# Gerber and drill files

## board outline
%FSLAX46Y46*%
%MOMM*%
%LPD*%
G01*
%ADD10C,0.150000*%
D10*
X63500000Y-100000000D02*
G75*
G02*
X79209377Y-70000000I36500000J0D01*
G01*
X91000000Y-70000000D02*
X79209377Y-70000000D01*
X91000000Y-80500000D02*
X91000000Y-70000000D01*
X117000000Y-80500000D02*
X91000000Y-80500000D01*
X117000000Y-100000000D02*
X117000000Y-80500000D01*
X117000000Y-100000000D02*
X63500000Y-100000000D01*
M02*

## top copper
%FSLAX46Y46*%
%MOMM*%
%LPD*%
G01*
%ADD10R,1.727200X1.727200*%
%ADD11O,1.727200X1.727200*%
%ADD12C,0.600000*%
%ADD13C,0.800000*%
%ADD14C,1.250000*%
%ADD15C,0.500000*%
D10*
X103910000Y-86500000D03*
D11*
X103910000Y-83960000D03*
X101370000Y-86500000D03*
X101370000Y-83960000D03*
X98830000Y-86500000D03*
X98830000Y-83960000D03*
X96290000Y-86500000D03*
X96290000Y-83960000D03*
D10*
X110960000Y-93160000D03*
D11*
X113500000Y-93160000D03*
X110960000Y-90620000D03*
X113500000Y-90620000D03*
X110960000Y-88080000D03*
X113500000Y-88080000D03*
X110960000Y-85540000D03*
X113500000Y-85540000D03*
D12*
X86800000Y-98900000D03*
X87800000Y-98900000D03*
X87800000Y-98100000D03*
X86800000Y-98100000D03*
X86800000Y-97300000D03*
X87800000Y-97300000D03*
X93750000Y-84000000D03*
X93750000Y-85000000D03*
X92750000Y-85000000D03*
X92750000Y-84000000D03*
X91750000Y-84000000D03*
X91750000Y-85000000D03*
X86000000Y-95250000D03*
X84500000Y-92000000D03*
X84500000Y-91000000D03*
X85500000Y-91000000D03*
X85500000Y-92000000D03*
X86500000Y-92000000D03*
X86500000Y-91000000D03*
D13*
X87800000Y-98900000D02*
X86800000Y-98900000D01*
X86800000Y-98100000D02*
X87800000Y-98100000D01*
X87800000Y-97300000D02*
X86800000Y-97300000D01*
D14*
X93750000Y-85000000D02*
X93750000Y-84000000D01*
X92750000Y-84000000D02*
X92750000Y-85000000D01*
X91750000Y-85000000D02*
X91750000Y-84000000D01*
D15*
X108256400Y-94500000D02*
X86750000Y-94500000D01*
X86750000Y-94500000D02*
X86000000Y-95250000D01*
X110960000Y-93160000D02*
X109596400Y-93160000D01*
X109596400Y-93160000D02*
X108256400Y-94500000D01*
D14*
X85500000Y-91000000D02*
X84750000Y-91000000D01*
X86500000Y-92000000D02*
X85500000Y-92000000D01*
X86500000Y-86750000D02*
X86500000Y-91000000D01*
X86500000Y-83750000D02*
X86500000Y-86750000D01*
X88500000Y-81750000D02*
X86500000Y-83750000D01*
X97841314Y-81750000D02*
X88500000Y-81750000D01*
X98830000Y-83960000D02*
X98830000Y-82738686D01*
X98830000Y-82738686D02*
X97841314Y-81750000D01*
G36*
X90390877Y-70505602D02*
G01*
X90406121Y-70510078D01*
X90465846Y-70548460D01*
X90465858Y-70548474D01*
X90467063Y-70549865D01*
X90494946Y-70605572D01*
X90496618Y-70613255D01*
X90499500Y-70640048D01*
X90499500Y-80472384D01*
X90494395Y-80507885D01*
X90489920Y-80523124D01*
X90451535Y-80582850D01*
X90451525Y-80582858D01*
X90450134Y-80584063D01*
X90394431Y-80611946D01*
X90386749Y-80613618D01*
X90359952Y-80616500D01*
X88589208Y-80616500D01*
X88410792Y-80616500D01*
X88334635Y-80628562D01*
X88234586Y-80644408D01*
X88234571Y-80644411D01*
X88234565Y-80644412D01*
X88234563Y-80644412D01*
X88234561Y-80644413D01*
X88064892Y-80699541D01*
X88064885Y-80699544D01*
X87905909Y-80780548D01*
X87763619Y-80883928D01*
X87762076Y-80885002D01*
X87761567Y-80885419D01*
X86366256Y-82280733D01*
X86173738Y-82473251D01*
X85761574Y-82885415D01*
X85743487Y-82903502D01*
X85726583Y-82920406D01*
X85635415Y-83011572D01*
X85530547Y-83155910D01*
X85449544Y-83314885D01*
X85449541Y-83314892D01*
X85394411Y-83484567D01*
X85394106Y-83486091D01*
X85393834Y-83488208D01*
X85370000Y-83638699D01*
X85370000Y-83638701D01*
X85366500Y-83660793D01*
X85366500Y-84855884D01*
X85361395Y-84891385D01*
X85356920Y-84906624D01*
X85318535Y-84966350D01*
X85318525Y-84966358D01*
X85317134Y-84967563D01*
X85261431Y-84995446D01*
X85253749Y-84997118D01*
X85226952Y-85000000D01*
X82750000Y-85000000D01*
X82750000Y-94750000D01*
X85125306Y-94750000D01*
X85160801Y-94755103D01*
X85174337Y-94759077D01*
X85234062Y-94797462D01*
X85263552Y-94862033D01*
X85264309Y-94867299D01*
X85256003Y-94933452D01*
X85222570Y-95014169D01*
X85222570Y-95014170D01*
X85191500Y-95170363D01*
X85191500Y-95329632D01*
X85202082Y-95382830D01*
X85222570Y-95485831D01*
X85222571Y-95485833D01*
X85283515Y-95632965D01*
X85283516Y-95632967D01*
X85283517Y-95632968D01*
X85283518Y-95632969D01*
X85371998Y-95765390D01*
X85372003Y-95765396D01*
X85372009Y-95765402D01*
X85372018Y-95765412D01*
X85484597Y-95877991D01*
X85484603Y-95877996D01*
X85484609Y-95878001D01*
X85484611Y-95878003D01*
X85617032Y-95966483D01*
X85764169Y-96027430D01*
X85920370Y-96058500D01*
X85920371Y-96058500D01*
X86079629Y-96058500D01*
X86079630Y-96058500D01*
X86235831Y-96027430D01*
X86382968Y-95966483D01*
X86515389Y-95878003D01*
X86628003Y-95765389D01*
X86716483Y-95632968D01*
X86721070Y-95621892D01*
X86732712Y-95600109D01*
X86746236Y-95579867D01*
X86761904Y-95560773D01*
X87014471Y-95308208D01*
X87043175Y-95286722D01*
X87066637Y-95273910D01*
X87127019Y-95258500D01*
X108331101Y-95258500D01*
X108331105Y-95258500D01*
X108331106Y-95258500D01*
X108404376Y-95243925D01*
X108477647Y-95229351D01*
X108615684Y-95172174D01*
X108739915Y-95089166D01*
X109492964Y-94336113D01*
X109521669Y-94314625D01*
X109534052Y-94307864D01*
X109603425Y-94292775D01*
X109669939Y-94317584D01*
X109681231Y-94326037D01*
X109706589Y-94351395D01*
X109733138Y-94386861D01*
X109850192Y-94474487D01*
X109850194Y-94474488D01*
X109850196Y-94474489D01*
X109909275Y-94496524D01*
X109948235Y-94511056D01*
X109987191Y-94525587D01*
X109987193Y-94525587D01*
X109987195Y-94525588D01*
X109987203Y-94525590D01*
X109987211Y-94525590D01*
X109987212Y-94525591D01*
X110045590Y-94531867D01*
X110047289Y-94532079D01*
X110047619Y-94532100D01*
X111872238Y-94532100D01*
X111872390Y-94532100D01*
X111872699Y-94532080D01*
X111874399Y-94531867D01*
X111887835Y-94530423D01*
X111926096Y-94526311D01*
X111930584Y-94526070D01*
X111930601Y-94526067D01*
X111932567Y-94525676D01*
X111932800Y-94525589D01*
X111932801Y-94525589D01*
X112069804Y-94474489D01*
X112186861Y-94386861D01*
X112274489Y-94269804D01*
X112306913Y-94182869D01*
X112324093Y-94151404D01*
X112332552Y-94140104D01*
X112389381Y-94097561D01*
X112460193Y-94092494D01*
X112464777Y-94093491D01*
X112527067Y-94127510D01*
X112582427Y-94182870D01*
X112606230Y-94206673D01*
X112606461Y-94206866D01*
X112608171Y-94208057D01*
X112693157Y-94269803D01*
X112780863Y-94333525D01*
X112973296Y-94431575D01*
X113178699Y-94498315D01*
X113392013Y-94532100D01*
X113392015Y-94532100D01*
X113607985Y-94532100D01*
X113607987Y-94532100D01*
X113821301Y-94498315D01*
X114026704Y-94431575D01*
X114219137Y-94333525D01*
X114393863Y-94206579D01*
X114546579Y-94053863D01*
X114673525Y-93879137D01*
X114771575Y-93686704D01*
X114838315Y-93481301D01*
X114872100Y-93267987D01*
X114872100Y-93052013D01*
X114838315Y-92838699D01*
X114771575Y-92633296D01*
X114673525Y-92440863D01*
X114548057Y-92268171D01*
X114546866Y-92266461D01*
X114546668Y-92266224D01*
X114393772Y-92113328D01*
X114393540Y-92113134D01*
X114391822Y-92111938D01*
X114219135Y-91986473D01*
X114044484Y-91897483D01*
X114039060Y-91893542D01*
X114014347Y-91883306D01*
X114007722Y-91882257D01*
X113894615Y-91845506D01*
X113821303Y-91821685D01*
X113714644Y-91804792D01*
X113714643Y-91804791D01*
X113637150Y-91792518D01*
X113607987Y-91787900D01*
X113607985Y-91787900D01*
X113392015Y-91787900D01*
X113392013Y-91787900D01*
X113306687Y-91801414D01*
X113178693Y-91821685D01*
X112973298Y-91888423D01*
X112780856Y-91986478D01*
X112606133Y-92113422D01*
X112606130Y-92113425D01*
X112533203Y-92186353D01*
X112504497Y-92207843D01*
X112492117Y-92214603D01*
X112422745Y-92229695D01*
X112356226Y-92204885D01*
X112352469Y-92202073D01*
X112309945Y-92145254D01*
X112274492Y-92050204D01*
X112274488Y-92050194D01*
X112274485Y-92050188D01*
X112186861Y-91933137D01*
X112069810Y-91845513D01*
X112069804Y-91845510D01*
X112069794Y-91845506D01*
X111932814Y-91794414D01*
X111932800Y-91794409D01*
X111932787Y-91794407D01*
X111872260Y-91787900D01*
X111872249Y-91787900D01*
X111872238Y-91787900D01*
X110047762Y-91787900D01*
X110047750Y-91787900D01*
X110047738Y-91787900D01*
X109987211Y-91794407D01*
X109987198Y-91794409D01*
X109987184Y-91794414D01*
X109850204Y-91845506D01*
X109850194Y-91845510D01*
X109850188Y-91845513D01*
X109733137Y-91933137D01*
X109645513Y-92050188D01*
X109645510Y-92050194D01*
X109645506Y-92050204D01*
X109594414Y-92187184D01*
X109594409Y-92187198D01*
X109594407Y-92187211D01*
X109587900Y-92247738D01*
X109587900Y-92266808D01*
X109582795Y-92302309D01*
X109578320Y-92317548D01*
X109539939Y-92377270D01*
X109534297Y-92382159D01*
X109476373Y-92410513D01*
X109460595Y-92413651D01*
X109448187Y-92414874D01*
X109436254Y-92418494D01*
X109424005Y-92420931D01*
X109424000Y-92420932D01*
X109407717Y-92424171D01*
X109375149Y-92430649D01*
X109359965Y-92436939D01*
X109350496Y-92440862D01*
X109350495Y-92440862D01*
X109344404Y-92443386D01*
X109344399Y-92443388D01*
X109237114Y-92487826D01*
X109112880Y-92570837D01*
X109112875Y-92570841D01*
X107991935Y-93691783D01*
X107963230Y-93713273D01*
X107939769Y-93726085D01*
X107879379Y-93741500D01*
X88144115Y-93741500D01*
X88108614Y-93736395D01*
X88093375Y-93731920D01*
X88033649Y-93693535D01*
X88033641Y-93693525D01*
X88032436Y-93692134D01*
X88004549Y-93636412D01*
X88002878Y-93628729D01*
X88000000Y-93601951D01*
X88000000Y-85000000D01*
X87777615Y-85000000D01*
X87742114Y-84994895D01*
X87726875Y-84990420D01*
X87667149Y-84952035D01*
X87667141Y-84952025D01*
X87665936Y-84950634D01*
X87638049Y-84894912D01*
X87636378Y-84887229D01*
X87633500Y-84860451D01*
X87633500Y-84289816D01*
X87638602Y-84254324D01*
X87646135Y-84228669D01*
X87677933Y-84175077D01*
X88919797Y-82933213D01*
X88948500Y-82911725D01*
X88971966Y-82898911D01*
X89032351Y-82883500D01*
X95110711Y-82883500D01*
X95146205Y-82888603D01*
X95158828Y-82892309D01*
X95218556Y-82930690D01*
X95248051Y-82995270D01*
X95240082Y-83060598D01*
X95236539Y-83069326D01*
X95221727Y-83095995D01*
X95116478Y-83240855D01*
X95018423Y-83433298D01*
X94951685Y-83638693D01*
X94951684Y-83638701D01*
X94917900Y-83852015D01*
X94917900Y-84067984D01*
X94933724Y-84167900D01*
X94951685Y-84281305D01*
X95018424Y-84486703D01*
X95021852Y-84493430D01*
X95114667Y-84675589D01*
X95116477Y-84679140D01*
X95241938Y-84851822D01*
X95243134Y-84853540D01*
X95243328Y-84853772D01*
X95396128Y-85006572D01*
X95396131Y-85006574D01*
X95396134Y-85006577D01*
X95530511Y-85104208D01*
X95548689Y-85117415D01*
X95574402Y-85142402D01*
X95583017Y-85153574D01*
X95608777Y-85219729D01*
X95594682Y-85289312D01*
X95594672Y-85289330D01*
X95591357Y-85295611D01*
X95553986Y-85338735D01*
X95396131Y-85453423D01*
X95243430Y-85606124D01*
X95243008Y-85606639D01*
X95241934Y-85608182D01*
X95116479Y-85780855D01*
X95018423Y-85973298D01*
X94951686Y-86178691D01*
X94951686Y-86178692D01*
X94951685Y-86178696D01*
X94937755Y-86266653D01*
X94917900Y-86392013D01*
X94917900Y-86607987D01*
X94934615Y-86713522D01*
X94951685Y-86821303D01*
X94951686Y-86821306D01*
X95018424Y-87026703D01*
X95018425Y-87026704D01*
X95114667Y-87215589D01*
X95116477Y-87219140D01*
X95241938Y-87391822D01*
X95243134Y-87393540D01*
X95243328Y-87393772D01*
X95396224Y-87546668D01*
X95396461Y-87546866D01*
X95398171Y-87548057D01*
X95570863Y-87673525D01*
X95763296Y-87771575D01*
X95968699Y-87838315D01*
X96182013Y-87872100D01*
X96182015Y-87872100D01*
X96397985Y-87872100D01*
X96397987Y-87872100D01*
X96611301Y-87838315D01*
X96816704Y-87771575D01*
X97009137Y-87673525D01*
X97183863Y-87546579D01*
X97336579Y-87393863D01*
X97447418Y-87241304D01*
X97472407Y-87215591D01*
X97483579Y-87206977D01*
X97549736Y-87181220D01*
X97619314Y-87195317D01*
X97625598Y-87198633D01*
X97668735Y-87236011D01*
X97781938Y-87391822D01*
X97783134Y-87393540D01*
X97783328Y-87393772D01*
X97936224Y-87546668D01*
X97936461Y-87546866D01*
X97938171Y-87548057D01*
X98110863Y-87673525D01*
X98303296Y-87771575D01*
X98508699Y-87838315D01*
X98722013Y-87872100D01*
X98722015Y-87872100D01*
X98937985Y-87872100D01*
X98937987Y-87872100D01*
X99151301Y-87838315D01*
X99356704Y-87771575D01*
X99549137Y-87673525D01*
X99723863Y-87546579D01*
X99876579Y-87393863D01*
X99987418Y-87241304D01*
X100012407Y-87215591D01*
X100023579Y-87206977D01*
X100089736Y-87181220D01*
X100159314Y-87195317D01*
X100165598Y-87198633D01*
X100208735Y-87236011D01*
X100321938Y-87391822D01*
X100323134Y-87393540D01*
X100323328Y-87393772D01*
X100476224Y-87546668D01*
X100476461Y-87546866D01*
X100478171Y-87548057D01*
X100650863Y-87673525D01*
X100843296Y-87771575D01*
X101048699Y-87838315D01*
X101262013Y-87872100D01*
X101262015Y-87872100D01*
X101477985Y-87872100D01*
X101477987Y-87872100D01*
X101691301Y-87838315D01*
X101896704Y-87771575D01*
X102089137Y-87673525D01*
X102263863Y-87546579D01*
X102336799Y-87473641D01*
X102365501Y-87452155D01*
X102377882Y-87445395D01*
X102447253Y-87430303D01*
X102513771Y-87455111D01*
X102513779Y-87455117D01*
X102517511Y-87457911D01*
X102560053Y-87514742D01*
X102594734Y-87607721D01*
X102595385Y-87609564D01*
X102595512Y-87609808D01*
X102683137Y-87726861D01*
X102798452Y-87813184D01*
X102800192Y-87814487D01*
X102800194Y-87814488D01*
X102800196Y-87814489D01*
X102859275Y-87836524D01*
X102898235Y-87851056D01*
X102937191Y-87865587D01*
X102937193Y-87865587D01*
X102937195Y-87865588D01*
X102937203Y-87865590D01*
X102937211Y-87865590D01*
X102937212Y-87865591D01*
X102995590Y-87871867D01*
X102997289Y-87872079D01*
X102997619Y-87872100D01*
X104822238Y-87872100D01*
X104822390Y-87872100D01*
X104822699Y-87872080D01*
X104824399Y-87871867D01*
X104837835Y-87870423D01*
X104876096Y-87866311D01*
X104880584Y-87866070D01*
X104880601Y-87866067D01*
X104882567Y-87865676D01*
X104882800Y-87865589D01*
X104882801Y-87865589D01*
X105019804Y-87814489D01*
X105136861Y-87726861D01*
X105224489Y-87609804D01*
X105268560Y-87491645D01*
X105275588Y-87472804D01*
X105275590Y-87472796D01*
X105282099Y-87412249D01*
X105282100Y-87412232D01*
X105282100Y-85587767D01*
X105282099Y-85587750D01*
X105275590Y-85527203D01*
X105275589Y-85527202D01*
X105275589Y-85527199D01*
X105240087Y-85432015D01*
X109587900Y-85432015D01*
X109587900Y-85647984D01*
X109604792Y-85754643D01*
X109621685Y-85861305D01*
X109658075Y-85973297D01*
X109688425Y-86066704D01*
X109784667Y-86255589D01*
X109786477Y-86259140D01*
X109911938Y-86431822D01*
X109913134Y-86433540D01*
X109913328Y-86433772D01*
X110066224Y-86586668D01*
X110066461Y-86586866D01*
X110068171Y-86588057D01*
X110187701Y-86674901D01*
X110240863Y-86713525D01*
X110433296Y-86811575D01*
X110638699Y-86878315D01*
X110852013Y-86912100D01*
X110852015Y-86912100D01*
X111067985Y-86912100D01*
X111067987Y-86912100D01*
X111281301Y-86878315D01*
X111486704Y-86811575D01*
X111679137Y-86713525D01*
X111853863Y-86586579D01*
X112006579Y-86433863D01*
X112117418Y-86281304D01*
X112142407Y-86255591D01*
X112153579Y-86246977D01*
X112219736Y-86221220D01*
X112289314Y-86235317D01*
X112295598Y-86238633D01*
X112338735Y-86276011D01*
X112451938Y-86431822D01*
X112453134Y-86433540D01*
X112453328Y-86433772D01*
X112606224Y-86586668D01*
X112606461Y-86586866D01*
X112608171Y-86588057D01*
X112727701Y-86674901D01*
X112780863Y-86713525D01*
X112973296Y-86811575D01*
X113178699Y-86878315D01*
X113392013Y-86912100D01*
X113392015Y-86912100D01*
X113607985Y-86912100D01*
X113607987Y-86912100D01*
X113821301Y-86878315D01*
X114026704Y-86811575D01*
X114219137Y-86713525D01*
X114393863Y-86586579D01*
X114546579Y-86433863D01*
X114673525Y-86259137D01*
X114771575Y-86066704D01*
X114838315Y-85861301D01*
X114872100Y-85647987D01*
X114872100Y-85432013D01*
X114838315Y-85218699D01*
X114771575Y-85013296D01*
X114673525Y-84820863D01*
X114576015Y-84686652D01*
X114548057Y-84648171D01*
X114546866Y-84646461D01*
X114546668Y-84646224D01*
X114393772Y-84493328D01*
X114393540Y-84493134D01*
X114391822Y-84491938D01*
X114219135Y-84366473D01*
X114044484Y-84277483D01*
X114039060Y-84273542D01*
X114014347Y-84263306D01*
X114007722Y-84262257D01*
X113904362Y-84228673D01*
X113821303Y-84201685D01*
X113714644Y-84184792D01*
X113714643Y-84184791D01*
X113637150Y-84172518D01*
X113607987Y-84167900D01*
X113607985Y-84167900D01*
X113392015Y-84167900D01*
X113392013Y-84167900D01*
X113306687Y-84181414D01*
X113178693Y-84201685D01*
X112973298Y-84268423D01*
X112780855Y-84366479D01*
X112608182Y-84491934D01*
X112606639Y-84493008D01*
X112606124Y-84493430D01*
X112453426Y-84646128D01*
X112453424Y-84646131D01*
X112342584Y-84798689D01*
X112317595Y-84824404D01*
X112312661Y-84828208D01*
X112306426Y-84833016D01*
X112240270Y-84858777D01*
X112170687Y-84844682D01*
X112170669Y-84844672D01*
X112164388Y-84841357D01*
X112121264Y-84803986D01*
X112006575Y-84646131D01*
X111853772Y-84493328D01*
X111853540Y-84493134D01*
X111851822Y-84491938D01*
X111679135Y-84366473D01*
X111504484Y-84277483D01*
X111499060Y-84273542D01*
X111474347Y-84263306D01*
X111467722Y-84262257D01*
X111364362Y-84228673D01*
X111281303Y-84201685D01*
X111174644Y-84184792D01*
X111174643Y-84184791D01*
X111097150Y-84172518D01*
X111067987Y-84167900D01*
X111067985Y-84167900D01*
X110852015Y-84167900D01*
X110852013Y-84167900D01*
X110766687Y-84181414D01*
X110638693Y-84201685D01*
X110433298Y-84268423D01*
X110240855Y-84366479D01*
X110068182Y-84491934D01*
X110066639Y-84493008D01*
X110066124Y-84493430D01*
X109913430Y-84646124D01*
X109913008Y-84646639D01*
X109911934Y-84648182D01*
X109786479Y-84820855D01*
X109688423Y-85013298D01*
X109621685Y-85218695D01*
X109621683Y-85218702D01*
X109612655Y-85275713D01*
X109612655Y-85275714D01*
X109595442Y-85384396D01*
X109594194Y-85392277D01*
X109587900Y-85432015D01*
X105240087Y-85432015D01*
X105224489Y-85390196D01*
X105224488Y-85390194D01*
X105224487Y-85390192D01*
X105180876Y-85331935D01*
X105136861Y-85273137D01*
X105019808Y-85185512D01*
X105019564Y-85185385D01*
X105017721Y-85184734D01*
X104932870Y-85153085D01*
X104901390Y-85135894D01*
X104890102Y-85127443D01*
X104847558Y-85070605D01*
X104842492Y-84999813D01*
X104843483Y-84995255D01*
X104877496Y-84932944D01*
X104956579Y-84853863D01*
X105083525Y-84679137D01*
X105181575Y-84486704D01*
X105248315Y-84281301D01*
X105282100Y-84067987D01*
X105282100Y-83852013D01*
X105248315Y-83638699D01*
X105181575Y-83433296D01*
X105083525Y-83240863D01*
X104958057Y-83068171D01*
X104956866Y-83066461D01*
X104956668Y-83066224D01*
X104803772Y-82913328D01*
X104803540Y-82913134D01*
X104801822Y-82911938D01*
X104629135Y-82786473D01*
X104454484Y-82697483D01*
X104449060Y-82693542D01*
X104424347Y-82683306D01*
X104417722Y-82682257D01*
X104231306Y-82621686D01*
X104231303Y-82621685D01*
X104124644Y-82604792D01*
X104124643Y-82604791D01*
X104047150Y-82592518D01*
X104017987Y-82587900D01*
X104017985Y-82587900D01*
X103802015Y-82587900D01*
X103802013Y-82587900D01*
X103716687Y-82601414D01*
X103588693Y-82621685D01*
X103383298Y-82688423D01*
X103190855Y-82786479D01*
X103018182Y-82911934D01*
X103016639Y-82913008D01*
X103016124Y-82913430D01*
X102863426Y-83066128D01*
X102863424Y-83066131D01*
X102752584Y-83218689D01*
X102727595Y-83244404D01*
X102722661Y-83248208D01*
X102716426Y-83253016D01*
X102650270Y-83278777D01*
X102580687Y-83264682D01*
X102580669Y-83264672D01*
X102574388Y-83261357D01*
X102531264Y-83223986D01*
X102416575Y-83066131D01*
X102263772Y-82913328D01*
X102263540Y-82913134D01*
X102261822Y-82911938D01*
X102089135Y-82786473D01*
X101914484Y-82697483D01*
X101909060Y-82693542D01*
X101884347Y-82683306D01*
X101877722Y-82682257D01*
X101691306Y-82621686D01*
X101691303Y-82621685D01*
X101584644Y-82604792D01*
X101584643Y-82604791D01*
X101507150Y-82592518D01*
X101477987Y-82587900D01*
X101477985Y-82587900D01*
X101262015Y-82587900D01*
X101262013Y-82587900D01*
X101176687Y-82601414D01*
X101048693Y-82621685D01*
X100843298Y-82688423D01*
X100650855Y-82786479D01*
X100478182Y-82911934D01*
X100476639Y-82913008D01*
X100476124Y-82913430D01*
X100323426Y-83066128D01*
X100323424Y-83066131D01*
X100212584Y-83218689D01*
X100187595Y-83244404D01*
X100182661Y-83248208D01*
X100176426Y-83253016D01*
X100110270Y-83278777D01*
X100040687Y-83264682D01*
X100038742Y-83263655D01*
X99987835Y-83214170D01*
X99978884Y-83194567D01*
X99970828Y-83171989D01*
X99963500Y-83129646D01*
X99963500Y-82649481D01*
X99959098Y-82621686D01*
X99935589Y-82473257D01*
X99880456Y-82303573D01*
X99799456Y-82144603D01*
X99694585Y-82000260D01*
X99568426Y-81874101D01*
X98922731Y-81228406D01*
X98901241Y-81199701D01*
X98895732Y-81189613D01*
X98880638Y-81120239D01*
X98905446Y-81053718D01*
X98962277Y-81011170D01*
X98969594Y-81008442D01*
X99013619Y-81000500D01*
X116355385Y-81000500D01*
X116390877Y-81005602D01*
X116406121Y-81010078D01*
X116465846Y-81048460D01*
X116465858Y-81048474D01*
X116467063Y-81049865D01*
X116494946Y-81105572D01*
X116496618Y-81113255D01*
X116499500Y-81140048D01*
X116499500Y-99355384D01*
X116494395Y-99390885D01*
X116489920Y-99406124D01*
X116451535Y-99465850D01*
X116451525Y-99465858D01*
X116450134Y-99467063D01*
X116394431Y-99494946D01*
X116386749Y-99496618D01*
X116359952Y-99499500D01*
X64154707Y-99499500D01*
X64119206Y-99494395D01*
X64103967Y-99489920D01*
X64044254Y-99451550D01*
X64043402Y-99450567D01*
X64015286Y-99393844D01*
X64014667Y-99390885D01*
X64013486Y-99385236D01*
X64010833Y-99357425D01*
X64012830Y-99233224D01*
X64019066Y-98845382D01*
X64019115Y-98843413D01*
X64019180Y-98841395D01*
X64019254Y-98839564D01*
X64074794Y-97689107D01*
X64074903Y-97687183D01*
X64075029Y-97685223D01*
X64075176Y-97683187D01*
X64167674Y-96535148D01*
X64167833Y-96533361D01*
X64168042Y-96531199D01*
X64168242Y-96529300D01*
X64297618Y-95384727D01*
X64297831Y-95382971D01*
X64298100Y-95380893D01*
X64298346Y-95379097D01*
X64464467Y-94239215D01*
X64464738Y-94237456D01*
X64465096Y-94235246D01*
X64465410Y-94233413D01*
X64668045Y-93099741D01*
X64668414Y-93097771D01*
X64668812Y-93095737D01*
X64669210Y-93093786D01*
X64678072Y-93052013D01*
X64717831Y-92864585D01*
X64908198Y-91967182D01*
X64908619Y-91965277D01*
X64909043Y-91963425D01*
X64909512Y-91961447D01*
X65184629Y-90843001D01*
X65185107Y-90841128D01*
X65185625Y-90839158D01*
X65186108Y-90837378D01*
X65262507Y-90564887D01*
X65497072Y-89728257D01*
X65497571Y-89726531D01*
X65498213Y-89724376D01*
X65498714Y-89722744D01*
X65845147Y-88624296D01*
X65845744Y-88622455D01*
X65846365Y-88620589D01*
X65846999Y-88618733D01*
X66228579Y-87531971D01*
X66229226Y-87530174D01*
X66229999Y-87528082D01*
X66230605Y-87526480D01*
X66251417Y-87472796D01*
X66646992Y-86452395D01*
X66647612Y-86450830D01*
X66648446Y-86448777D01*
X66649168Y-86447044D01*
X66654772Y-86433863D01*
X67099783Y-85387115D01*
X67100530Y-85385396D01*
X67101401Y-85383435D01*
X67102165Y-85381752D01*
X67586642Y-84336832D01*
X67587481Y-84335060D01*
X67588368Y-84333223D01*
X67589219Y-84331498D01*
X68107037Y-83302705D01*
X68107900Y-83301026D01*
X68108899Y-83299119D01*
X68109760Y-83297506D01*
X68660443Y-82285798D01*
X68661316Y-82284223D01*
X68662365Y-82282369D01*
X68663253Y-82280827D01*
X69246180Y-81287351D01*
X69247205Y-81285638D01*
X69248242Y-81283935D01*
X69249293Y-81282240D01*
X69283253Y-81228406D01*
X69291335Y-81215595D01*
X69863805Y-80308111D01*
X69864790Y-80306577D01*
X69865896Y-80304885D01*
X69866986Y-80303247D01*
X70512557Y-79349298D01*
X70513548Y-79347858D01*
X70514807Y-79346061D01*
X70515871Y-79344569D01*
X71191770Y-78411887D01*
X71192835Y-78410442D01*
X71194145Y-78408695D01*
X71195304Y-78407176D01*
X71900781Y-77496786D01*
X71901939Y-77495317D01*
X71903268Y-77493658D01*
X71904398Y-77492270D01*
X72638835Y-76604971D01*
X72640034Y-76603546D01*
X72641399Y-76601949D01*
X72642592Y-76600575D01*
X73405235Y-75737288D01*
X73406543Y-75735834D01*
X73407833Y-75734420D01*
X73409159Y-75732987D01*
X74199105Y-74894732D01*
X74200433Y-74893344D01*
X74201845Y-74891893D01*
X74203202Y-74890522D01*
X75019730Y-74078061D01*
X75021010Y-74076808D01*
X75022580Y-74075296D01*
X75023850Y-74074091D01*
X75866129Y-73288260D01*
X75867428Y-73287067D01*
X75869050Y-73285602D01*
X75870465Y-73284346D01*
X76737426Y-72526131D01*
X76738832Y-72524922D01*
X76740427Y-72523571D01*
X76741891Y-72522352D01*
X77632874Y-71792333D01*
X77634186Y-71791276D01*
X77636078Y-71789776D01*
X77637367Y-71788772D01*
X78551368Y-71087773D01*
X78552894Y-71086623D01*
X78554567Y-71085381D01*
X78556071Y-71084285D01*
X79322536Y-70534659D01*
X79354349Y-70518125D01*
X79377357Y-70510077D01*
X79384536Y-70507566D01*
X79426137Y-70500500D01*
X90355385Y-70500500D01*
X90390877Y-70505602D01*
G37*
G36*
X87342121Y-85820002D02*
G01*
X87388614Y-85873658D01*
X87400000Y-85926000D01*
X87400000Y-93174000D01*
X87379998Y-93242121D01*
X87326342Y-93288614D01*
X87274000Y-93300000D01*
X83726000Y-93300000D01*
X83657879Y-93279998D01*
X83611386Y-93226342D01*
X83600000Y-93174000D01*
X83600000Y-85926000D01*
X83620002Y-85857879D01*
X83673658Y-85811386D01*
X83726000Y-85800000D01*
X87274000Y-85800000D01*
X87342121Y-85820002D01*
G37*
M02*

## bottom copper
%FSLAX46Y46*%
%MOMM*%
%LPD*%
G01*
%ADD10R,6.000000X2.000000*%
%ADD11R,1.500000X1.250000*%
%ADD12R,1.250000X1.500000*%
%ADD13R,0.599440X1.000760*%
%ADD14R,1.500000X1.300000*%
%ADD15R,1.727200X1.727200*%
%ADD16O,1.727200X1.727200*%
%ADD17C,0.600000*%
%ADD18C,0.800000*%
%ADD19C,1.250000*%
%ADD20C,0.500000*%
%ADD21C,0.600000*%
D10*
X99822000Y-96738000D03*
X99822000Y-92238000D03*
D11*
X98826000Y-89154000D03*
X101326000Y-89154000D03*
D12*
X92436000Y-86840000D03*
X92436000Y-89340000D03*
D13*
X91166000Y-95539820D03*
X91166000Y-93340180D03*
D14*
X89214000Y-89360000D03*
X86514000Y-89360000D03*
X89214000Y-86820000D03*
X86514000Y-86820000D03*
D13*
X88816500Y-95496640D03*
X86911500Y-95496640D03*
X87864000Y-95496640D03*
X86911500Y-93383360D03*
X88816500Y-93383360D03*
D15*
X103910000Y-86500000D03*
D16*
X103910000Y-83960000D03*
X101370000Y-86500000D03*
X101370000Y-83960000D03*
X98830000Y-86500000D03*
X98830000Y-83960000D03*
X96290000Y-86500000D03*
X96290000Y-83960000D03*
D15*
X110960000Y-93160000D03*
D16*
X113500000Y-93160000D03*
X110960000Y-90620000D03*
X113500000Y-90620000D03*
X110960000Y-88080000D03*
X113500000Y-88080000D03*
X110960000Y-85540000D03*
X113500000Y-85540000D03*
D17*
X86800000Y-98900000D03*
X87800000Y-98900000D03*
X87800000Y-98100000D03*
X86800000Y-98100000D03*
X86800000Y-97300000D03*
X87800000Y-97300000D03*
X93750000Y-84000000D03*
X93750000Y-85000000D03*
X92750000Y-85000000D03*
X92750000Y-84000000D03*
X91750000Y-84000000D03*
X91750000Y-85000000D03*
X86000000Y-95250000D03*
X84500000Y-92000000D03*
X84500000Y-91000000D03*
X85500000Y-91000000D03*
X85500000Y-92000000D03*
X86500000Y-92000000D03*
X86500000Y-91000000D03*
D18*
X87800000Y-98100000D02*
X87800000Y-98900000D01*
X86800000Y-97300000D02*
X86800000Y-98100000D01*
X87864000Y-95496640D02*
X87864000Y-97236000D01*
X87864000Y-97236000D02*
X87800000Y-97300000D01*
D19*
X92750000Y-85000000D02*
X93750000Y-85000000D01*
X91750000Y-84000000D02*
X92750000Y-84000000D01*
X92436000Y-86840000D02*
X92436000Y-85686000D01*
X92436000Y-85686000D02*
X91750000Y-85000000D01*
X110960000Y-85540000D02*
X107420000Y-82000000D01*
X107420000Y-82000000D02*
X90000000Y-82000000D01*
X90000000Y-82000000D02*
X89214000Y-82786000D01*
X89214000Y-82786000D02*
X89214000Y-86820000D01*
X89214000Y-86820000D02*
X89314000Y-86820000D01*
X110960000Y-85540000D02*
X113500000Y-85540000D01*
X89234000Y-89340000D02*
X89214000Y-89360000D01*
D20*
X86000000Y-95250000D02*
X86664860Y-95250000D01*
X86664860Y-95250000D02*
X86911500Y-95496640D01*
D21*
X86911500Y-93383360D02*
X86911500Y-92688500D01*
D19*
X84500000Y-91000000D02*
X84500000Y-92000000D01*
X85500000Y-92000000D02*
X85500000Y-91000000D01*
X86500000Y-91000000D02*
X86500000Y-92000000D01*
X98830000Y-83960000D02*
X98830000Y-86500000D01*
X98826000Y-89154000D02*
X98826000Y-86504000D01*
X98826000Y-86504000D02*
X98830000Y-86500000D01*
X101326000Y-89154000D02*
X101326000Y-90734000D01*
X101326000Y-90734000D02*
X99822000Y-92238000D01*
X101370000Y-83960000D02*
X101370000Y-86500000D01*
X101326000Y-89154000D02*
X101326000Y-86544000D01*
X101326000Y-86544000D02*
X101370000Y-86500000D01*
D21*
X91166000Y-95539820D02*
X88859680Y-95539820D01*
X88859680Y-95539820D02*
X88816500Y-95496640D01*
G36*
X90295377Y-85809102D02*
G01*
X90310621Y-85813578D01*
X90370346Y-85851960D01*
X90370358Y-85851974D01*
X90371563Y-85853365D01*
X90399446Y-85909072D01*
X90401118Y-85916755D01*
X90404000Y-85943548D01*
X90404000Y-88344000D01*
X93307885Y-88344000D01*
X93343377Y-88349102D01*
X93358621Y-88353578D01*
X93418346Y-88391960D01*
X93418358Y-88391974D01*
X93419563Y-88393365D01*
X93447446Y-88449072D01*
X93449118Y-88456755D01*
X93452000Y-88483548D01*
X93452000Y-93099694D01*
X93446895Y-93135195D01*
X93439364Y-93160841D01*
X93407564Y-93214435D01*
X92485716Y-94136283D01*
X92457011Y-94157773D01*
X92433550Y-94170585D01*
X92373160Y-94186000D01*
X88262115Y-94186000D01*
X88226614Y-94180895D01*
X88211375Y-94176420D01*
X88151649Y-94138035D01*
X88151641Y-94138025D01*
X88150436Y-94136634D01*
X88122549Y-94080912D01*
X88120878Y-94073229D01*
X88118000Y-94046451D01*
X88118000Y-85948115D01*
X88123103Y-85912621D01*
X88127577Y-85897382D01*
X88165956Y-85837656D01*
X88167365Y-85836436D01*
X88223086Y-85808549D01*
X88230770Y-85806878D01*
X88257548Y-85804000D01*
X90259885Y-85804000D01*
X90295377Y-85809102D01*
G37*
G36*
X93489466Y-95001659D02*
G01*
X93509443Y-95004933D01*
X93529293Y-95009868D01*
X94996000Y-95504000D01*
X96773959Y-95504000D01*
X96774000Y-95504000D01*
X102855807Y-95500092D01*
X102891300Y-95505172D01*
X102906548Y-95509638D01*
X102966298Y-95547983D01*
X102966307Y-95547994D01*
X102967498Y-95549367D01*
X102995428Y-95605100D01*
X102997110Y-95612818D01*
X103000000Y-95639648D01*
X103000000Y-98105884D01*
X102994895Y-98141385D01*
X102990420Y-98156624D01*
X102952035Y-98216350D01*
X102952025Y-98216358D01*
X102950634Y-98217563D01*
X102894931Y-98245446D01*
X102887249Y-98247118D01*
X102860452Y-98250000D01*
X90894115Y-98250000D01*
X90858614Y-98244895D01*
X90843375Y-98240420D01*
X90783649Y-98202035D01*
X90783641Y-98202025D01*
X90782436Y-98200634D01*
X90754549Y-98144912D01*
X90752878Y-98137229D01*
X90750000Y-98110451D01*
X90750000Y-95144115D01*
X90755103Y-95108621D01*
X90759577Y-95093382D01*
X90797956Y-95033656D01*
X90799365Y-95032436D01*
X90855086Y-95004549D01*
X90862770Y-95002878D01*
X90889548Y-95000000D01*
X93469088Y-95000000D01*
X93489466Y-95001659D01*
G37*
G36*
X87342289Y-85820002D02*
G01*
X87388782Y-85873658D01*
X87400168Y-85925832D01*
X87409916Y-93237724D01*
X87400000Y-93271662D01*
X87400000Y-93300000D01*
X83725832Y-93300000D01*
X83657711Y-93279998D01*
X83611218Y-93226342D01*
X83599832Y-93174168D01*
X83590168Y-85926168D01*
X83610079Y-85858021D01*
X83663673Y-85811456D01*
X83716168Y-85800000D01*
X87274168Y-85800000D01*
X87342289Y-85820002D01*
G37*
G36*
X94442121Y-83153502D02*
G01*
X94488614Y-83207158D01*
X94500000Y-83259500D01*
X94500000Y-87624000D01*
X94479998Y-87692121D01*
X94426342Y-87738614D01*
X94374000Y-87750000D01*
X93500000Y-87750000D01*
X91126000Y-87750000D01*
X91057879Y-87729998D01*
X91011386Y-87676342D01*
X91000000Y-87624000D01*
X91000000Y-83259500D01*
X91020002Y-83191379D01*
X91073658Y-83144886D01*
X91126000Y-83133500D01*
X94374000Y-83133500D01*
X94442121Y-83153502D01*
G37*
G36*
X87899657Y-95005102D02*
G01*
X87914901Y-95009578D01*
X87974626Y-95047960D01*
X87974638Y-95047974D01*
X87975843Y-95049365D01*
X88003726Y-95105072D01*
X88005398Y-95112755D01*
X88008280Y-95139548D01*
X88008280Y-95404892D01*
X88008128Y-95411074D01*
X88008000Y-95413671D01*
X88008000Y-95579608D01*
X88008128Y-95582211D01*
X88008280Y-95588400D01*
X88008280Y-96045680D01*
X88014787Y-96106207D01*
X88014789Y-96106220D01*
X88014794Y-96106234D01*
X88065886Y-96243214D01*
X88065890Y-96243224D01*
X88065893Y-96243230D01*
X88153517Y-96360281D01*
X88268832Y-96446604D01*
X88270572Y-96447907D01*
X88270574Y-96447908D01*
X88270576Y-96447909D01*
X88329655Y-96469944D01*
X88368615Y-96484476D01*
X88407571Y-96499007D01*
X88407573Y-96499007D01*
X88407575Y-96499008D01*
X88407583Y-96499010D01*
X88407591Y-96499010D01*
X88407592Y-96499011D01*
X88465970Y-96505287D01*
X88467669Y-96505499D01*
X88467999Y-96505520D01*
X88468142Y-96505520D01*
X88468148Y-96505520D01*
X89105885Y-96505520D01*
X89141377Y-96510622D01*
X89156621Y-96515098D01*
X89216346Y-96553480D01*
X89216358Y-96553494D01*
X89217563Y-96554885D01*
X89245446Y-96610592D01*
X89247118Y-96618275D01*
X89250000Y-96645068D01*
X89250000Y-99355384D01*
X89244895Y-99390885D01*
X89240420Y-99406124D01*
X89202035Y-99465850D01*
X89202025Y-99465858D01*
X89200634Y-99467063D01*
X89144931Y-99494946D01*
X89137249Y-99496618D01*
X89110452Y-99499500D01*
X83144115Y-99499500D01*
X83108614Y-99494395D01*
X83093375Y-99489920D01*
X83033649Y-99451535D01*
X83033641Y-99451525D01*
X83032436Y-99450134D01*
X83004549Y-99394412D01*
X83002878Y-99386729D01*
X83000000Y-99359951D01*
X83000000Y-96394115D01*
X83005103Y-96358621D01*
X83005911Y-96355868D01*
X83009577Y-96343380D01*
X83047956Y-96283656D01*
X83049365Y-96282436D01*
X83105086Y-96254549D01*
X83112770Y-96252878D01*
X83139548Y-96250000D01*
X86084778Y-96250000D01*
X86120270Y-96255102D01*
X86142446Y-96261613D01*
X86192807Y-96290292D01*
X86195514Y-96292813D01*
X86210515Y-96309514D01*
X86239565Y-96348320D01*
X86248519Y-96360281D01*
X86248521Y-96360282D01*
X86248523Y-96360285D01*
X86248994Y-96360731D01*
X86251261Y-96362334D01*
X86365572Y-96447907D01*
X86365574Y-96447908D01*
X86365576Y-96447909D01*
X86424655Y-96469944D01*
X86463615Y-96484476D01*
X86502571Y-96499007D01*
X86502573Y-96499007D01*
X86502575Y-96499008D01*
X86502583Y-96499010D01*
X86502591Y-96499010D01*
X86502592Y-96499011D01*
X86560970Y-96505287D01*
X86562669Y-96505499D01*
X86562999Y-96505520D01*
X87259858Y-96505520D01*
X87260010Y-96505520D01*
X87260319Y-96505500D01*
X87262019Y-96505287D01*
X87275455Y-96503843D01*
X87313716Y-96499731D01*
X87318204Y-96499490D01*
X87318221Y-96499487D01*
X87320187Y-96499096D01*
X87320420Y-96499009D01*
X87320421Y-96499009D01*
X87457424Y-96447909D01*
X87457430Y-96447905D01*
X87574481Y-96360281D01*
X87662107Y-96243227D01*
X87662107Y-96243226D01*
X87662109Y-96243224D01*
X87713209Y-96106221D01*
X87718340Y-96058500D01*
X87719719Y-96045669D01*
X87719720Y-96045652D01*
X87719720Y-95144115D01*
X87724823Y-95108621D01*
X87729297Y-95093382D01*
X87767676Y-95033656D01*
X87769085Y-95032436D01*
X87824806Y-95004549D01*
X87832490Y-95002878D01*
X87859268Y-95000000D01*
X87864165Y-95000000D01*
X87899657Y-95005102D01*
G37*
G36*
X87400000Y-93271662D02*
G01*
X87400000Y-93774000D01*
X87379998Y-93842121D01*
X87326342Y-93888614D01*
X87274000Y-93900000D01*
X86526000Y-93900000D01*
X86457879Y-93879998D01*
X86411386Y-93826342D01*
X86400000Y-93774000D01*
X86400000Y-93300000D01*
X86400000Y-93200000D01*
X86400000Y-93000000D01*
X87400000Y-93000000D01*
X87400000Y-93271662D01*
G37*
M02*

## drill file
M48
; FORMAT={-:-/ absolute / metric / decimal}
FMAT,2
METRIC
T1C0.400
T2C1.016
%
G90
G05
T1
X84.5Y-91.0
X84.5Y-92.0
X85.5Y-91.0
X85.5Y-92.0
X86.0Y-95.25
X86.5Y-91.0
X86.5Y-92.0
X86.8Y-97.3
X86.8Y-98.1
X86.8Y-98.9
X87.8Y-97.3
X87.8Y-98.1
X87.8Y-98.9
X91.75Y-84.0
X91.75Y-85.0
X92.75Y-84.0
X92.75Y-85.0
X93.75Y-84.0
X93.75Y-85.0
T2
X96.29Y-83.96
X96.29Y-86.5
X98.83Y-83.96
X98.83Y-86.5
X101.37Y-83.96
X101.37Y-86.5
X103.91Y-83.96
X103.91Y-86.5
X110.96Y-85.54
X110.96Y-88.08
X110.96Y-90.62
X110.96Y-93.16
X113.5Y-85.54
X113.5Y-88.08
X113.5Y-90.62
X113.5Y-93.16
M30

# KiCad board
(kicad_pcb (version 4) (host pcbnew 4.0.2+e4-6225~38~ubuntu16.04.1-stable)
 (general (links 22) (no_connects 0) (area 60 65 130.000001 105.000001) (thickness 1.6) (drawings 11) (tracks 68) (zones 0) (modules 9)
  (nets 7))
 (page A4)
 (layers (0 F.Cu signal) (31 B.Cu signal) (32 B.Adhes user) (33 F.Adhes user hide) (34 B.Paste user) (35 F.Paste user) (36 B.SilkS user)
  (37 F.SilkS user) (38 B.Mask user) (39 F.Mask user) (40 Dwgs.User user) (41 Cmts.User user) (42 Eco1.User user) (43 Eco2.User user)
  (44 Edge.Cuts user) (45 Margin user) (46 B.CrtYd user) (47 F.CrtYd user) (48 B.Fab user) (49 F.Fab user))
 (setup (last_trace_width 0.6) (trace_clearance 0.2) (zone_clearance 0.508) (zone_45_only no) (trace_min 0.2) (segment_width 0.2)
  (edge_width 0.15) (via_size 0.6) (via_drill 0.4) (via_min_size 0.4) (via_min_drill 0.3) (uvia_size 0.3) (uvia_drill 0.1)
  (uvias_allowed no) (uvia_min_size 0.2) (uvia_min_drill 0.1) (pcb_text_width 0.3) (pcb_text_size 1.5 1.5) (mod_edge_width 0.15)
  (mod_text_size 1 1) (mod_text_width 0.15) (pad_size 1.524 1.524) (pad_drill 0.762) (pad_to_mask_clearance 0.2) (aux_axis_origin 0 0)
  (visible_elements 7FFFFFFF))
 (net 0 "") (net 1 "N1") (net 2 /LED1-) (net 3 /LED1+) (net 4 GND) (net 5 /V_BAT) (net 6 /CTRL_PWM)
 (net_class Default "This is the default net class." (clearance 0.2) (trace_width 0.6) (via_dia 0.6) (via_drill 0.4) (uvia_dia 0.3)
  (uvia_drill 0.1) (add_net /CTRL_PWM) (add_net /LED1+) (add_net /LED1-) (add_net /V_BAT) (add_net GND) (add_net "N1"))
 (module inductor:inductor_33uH (layer B.Cu) (at 99.822 94.488 90)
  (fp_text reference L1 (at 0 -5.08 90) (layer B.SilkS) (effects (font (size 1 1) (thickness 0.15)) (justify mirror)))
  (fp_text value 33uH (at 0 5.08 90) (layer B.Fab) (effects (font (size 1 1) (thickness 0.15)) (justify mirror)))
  (pad 1 smd rect (at -2.25 0 90) (size 2 6) (layers B.Cu B.Paste B.Mask) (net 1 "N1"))
  (pad 2 smd rect (at 2.25 0 90) (size 2 6) (layers B.Cu B.Paste B.Mask) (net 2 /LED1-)))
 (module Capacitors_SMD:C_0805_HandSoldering (layer B.Cu) (at 100.076 89.154)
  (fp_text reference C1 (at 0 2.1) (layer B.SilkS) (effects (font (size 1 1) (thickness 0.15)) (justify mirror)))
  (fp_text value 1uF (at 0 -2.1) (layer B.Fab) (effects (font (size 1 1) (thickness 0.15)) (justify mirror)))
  (pad 1 smd rect (at -1.25 0) (size 1.5 1.25) (layers B.Cu B.Paste B.Mask) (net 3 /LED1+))
  (pad 2 smd rect (at 1.25 0) (size 1.5 1.25) (layers B.Cu B.Paste B.Mask) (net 2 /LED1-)))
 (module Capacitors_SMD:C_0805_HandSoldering (layer B.Cu) (at 92.436 88.09 270)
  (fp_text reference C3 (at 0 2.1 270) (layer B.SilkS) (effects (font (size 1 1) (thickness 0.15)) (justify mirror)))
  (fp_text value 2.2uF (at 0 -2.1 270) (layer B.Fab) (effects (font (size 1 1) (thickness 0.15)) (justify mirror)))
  (pad 1 smd rect (at -1.25 0 270) (size 1.5 1.25) (layers B.Cu B.Paste B.Mask) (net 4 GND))
  (pad 2 smd rect (at 1.25 0 270) (size 1.5 1.25) (layers B.Cu B.Paste B.Mask) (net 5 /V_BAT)))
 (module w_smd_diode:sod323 (layer B.Cu) (at 91.166 94.44 270)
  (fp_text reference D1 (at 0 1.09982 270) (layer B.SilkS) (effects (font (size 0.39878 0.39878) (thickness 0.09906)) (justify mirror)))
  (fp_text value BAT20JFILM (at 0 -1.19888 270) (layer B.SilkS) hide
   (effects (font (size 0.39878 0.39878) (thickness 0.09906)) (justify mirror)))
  (pad 2 smd rect (at 1.09982 0 270) (size 1.00076 0.59944) (layers B.Cu B.Paste B.Mask) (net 1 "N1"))
  (pad 1 smd rect (at -1.09982 0 270) (size 1.00076 0.59944) (layers B.Cu B.Paste B.Mask) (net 5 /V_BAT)))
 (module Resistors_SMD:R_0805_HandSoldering (layer B.Cu) (at 87.864 89.36 180)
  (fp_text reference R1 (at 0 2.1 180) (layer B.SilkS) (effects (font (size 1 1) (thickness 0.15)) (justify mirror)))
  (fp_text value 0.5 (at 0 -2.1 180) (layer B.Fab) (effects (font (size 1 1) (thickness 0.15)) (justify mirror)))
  (pad 1 smd rect (at -1.35 0 180) (size 1.5 1.3) (layers B.Cu B.Paste B.Mask) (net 5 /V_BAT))
  (pad 2 smd rect (at 1.35 0 180) (size 1.5 1.3) (layers B.Cu B.Paste B.Mask) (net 3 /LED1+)))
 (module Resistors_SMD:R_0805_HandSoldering (layer B.Cu) (at 87.864 86.82 180)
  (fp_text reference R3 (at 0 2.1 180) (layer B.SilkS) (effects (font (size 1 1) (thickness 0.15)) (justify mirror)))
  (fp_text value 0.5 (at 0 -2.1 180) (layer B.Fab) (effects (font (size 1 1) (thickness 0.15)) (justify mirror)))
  (pad 1 smd rect (at -1.35 0 180) (size 1.5 1.3) (layers B.Cu B.Paste B.Mask) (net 5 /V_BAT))
  (pad 2 smd rect (at 1.35 0 180) (size 1.5 1.3) (layers B.Cu B.Paste B.Mask) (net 3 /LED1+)))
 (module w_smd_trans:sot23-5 (layer B.Cu) (at 87.864 94.44 180)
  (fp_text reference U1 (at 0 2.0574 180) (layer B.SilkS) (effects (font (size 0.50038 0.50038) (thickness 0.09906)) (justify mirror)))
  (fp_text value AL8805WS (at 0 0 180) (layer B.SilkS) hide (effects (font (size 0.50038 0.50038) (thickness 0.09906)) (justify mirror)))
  (pad 1 smd rect (at -0.9525 -1.05664 180) (size 0.59944 1.00076) (layers B.Cu B.Paste B.Mask) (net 1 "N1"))
  (pad 3 smd rect (at 0.9525 -1.05664 180) (size 0.59944 1.00076) (layers B.Cu B.Paste B.Mask) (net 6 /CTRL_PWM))
  (pad 2 smd rect (at 0 -1.05664 180) (size 0.59944 1.00076) (layers B.Cu B.Paste B.Mask) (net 4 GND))
  (pad 4 smd rect (at 0.9525 1.05664 180) (size 0.59944 1.00076) (layers B.Cu B.Paste B.Mask) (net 3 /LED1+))
  (pad 5 smd rect (at -0.9525 1.05664 180) (size 0.59944 1.00076) (layers B.Cu B.Paste B.Mask) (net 5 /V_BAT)))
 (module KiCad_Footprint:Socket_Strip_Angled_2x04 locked (layer F.Cu) (at 103.91 86.5 180)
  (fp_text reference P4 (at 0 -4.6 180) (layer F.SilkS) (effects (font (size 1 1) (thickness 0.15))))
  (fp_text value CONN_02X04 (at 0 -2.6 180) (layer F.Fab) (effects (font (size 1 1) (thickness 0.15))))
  (pad 1 thru_hole rect (at 0 0 180) (size 1.7272 1.7272) (drill 1.016) (layers *.Cu *.Mask F.SilkS))
  (pad 2 thru_hole oval (at 0 2.54 180) (size 1.7272 1.7272) (drill 1.016) (layers *.Cu *.Mask F.SilkS))
  (pad 3 thru_hole oval (at 2.54 0 180) (size 1.7272 1.7272) (drill 1.016) (layers *.Cu *.Mask F.SilkS) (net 2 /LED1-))
  (pad 4 thru_hole oval (at 2.54 2.54 180) (size 1.7272 1.7272) (drill 1.016) (layers *.Cu *.Mask F.SilkS) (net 2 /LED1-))
  (pad 5 thru_hole oval (at 5.08 0 180) (size 1.7272 1.7272) (drill 1.016) (layers *.Cu *.Mask F.SilkS) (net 3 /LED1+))
  (pad 6 thru_hole oval (at 5.08 2.54 180) (size 1.7272 1.7272) (drill 1.016) (layers *.Cu *.Mask F.SilkS) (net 3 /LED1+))
  (pad 7 thru_hole oval (at 7.62 0 180) (size 1.7272 1.7272) (drill 1.016) (layers *.Cu *.Mask F.SilkS))
  (pad 8 thru_hole oval (at 7.62 2.54 180) (size 1.7272 1.7272) (drill 1.016) (layers *.Cu *.Mask F.SilkS)))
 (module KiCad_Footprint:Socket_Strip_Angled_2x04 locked (layer F.Cu) (at 110.96 93.16 90)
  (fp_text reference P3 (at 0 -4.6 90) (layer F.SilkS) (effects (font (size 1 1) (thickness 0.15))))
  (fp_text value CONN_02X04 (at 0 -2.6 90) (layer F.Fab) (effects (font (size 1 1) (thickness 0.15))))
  (pad 1 thru_hole rect (at 0 0 90) (size 1.7272 1.7272) (drill 1.016) (layers *.Cu *.Mask F.SilkS) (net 6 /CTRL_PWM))
  (pad 2 thru_hole oval (at 0 2.54 90) (size 1.7272 1.7272) (drill 1.016) (layers *.Cu *.Mask F.SilkS))
  (pad 3 thru_hole oval (at 2.54 0 90) (size 1.7272 1.7272) (drill 1.016) (layers *.Cu *.Mask F.SilkS) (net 4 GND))
  (pad 4 thru_hole oval (at 2.54 2.54 90) (size 1.7272 1.7272) (drill 1.016) (layers *.Cu *.Mask F.SilkS) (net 4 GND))
  (pad 5 thru_hole oval (at 5.08 0 90) (size 1.7272 1.7272) (drill 1.016) (layers *.Cu *.Mask F.SilkS) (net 4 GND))
  (pad 6 thru_hole oval (at 5.08 2.54 90) (size 1.7272 1.7272) (drill 1.016) (layers *.Cu *.Mask F.SilkS) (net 4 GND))
  (pad 7 thru_hole oval (at 7.62 0 90) (size 1.7272 1.7272) (drill 1.016) (layers *.Cu *.Mask F.SilkS) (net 5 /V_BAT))
  (pad 8 thru_hole oval (at 7.62 2.54 90) (size 1.7272 1.7272) (drill 1.016) (layers *.Cu *.Mask F.SilkS) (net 5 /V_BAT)))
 (gr_arc (start 100 100) (end 63.5 100) (angle 55.27723707) (layer Edge.Cuts) (width 0.15))
 (gr_line (start 91 70) (end 79.209377 70) (layer Edge.Cuts) (width 0.15))
 (gr_line (start 91 80.5) (end 91 70) (layer Edge.Cuts) (width 0.15))
 (gr_line (start 117 80.5) (end 91 80.5) (layer Edge.Cuts) (width 0.15))
 (gr_line (start 117 100) (end 117 80.5) (layer Edge.Cuts) (width 0.15))
 (gr_line (start 117 100) (end 63.5 100) (layer Edge.Cuts) (width 0.15))
 (segment (start 87.8 98.9) (end 86.8 98.9) (width 0.8) (layer F.Cu) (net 4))
 (via (at 86.8 98.9) (size 0.6) (drill 0.4) (layers F.Cu B.Cu) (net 4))
 (segment (start 87.8 98.1) (end 87.8 98.9) (width 0.8) (layer B.Cu) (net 4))
 (via (at 87.8 98.9) (size 0.6) (drill 0.4) (layers F.Cu B.Cu) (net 4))
 (segment (start 86.8 98.1) (end 87.8 98.1) (width 0.8) (layer F.Cu) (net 4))
 (via (at 87.8 98.1) (size 0.6) (drill 0.4) (layers F.Cu B.Cu) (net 4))
 (segment (start 86.8 97.3) (end 86.8 98.1) (width 0.8) (layer B.Cu) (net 4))
 (via (at 86.8 98.1) (size 0.6) (drill 0.4) (layers F.Cu B.Cu) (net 4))
 (segment (start 87.8 97.3) (end 86.8 97.3) (width 0.8) (layer F.Cu) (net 4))
 (via (at 86.8 97.3) (size 0.6) (drill 0.4) (layers F.Cu B.Cu) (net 4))
 (segment (start 87.864 95.49664) (end 87.864 97.236) (width 0.8) (layer B.Cu) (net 4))
 (segment (start 87.864 97.236) (end 87.8 97.3) (width 0.8) (layer B.Cu) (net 4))
 (via (at 87.8 97.3) (size 0.6) (drill 0.4) (layers F.Cu B.Cu) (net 4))
 (segment (start 93.75 85) (end 93.75 84) (width 1.25) (layer F.Cu) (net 4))
 (via (at 93.75 84) (size 0.6) (drill 0.4) (layers F.Cu B.Cu) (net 4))
 (segment (start 92.75 85) (end 93.75 85) (width 1.25) (layer B.Cu) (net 4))
 (via (at 93.75 85) (size 0.6) (drill 0.4) (layers F.Cu B.Cu) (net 4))
 (segment (start 92.75 84) (end 92.75 85) (width 1.25) (layer F.Cu) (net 4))
 (via (at 92.75 85) (size 0.6) (drill 0.4) (layers F.Cu B.Cu) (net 4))
 (segment (start 91.75 84) (end 92.75 84) (width 1.25) (layer B.Cu) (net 4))
 (via (at 92.75 84) (size 0.6) (drill 0.4) (layers F.Cu B.Cu) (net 4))
 (segment (start 91.75 85) (end 91.75 84) (width 1.25) (layer F.Cu) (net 4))
 (via (at 91.75 84) (size 0.6) (drill 0.4) (layers F.Cu B.Cu) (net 4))
 (segment (start 92.436 86.84) (end 92.436 85.686) (width 1.25) (layer B.Cu) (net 4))
 (segment (start 92.436 85.686) (end 91.75 85) (width 1.25) (layer B.Cu) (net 4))
 (via (at 91.75 85) (size 0.6) (drill 0.4) (layers F.Cu B.Cu) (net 4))
 (segment (start 110.96 85.54) (end 107.42 82) (width 1.25) (layer B.Cu) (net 5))
 (segment (start 107.42 82) (end 90 82) (width 1.25) (layer B.Cu) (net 5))
 (segment (start 90 82) (end 89.214 82.786) (width 1.25) (layer B.Cu) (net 5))
 (segment (start 89.214 82.786) (end 89.214 86.82) (width 1.25) (layer B.Cu) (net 5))
 (segment (start 89.214 86.82) (end 89.314 86.82) (width 1.25) (layer B.Cu) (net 5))
 (segment (start 110.96 85.54) (end 113.5 85.54) (width 1.25) (layer B.Cu) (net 5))
 (segment (start 89.234 89.34) (end 89.214 89.36) (width 1.25) (layer B.Cu) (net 5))
 (segment (start 86 95.25) (end 86.66486 95.25) (width 0.5) (layer B.Cu) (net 6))
 (segment (start 86.66486 95.25) (end 86.9115 95.49664) (width 0.5) (layer B.Cu) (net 6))
 (segment (start 108.2564 94.5) (end 86.75 94.5) (width 0.5) (layer F.Cu) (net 6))
 (via (at 86 95.25) (size 0.6) (drill 0.4) (layers F.Cu B.Cu) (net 6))
 (segment (start 86.75 94.5) (end 86 95.25) (width 0.5) (layer F.Cu) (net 6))
 (segment (start 110.96 93.16) (end 109.5964 93.16) (width 0.5) (layer F.Cu) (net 6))
 (segment (start 109.5964 93.16) (end 108.2564 94.5) (width 0.5) (layer F.Cu) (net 6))
 (segment (start 86.9115 93.38336) (end 86.9115 92.6885) (width 0.6) (layer B.Cu) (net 3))
 (segment (start 84.5 91) (end 84.5 92) (width 1.25) (layer B.Cu) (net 3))
 (via (at 84.5 92) (size 0.6) (drill 0.4) (layers F.Cu B.Cu) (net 3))
 (segment (start 85.5 91) (end 84.75 91) (width 1.25) (layer F.Cu) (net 3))
 (via (at 84.5 91) (size 0.6) (drill 0.4) (layers F.Cu B.Cu) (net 3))
 (segment (start 85.5 92) (end 85.5 91) (width 1.25) (layer B.Cu) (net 3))
 (via (at 85.5 91) (size 0.6) (drill 0.4) (layers F.Cu B.Cu) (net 3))
 (segment (start 86.5 92) (end 85.5 92) (width 1.25) (layer F.Cu) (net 3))
 (via (at 85.5 92) (size 0.6) (drill 0.4) (layers F.Cu B.Cu) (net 3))
 (segment (start 86.5 91) (end 86.5 92) (width 1.25) (layer B.Cu) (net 3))
 (via (at 86.5 92) (size 0.6) (drill 0.4) (layers F.Cu B.Cu) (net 3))
 (segment (start 86.5 86.75) (end 86.5 91) (width 1.25) (layer F.Cu) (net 3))
 (via (at 86.5 91) (size 0.6) (drill 0.4) (layers F.Cu B.Cu) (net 3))
 (segment (start 86.5 83.75) (end 86.5 86.75) (width 1.25) (layer F.Cu) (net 3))
 (segment (start 88.5 81.75) (end 86.5 83.75) (width 1.25) (layer F.Cu) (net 3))
 (segment (start 97.841314 81.75) (end 88.5 81.75) (width 1.25) (layer F.Cu) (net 3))
 (segment (start 98.83 83.96) (end 98.83 82.738686) (width 1.25) (layer F.Cu) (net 3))
 (segment (start 98.83 82.738686) (end 97.841314 81.75) (width 1.25) (layer F.Cu) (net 3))
 (segment (start 98.83 83.96) (end 98.83 86.5) (width 1.25) (layer B.Cu) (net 3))
 (segment (start 98.826 89.154) (end 98.826 86.504) (width 1.25) (layer B.Cu) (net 3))
 (segment (start 98.826 86.504) (end 98.83 86.5) (width 1.25) (layer B.Cu) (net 3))
 (segment (start 101.326 89.154) (end 101.326 90.734) (width 1.25) (layer B.Cu) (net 2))
 (segment (start 101.326 90.734) (end 99.822 92.238) (width 1.25) (layer B.Cu) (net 2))
 (segment (start 101.37 83.96) (end 101.37 86.5) (width 1.25) (layer B.Cu) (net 2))
 (segment (start 101.326 89.154) (end 101.326 86.544) (width 1.25) (layer B.Cu) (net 2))
 (segment (start 101.326 86.544) (end 101.37 86.5) (width 1.25) (layer B.Cu) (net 2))
 (segment (start 91.166 95.53982) (end 88.85968 95.53982) (width 0.6) (layer B.Cu) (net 1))
 (segment (start 88.85968 95.53982) (end 88.8165 95.49664) (width 0.6) (layer B.Cu) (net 1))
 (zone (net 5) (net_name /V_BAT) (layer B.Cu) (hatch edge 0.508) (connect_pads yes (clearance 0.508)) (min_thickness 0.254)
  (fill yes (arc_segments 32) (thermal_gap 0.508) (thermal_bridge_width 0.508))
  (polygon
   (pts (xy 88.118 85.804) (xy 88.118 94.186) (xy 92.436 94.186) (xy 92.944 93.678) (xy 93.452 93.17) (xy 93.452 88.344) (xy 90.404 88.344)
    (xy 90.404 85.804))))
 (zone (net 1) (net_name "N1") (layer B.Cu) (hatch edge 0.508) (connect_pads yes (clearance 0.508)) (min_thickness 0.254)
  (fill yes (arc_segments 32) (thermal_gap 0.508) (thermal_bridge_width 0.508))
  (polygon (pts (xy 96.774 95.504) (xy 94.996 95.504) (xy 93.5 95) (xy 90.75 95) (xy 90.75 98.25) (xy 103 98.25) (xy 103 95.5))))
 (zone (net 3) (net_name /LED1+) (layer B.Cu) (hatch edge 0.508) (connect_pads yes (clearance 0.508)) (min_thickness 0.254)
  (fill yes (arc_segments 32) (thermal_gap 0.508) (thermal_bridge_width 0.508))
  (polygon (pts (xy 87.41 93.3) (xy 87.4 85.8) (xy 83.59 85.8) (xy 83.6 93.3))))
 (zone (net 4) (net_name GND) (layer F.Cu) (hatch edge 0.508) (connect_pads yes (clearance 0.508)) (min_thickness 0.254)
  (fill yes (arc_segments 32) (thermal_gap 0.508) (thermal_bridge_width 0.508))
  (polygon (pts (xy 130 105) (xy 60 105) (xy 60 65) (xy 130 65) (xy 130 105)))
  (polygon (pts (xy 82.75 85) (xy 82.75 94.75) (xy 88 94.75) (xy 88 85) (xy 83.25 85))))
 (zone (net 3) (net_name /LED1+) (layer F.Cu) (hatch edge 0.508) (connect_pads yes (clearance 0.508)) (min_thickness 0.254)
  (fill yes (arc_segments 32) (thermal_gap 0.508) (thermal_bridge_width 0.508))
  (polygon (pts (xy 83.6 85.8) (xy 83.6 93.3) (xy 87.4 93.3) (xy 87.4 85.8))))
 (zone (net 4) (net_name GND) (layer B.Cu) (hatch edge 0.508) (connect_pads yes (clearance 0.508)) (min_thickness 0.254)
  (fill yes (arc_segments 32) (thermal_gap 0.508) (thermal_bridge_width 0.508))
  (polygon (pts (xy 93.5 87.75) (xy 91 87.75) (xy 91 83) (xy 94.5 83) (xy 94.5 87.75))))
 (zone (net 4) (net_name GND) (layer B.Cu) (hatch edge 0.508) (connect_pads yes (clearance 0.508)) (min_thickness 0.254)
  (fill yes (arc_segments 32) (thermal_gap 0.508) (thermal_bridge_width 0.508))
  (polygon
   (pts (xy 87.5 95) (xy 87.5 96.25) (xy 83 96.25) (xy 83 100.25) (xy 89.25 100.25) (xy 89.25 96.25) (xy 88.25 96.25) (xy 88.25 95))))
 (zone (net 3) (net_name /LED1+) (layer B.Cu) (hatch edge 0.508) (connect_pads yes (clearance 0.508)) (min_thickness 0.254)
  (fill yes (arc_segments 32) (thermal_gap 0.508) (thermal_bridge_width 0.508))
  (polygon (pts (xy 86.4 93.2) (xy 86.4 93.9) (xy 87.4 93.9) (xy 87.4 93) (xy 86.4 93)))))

